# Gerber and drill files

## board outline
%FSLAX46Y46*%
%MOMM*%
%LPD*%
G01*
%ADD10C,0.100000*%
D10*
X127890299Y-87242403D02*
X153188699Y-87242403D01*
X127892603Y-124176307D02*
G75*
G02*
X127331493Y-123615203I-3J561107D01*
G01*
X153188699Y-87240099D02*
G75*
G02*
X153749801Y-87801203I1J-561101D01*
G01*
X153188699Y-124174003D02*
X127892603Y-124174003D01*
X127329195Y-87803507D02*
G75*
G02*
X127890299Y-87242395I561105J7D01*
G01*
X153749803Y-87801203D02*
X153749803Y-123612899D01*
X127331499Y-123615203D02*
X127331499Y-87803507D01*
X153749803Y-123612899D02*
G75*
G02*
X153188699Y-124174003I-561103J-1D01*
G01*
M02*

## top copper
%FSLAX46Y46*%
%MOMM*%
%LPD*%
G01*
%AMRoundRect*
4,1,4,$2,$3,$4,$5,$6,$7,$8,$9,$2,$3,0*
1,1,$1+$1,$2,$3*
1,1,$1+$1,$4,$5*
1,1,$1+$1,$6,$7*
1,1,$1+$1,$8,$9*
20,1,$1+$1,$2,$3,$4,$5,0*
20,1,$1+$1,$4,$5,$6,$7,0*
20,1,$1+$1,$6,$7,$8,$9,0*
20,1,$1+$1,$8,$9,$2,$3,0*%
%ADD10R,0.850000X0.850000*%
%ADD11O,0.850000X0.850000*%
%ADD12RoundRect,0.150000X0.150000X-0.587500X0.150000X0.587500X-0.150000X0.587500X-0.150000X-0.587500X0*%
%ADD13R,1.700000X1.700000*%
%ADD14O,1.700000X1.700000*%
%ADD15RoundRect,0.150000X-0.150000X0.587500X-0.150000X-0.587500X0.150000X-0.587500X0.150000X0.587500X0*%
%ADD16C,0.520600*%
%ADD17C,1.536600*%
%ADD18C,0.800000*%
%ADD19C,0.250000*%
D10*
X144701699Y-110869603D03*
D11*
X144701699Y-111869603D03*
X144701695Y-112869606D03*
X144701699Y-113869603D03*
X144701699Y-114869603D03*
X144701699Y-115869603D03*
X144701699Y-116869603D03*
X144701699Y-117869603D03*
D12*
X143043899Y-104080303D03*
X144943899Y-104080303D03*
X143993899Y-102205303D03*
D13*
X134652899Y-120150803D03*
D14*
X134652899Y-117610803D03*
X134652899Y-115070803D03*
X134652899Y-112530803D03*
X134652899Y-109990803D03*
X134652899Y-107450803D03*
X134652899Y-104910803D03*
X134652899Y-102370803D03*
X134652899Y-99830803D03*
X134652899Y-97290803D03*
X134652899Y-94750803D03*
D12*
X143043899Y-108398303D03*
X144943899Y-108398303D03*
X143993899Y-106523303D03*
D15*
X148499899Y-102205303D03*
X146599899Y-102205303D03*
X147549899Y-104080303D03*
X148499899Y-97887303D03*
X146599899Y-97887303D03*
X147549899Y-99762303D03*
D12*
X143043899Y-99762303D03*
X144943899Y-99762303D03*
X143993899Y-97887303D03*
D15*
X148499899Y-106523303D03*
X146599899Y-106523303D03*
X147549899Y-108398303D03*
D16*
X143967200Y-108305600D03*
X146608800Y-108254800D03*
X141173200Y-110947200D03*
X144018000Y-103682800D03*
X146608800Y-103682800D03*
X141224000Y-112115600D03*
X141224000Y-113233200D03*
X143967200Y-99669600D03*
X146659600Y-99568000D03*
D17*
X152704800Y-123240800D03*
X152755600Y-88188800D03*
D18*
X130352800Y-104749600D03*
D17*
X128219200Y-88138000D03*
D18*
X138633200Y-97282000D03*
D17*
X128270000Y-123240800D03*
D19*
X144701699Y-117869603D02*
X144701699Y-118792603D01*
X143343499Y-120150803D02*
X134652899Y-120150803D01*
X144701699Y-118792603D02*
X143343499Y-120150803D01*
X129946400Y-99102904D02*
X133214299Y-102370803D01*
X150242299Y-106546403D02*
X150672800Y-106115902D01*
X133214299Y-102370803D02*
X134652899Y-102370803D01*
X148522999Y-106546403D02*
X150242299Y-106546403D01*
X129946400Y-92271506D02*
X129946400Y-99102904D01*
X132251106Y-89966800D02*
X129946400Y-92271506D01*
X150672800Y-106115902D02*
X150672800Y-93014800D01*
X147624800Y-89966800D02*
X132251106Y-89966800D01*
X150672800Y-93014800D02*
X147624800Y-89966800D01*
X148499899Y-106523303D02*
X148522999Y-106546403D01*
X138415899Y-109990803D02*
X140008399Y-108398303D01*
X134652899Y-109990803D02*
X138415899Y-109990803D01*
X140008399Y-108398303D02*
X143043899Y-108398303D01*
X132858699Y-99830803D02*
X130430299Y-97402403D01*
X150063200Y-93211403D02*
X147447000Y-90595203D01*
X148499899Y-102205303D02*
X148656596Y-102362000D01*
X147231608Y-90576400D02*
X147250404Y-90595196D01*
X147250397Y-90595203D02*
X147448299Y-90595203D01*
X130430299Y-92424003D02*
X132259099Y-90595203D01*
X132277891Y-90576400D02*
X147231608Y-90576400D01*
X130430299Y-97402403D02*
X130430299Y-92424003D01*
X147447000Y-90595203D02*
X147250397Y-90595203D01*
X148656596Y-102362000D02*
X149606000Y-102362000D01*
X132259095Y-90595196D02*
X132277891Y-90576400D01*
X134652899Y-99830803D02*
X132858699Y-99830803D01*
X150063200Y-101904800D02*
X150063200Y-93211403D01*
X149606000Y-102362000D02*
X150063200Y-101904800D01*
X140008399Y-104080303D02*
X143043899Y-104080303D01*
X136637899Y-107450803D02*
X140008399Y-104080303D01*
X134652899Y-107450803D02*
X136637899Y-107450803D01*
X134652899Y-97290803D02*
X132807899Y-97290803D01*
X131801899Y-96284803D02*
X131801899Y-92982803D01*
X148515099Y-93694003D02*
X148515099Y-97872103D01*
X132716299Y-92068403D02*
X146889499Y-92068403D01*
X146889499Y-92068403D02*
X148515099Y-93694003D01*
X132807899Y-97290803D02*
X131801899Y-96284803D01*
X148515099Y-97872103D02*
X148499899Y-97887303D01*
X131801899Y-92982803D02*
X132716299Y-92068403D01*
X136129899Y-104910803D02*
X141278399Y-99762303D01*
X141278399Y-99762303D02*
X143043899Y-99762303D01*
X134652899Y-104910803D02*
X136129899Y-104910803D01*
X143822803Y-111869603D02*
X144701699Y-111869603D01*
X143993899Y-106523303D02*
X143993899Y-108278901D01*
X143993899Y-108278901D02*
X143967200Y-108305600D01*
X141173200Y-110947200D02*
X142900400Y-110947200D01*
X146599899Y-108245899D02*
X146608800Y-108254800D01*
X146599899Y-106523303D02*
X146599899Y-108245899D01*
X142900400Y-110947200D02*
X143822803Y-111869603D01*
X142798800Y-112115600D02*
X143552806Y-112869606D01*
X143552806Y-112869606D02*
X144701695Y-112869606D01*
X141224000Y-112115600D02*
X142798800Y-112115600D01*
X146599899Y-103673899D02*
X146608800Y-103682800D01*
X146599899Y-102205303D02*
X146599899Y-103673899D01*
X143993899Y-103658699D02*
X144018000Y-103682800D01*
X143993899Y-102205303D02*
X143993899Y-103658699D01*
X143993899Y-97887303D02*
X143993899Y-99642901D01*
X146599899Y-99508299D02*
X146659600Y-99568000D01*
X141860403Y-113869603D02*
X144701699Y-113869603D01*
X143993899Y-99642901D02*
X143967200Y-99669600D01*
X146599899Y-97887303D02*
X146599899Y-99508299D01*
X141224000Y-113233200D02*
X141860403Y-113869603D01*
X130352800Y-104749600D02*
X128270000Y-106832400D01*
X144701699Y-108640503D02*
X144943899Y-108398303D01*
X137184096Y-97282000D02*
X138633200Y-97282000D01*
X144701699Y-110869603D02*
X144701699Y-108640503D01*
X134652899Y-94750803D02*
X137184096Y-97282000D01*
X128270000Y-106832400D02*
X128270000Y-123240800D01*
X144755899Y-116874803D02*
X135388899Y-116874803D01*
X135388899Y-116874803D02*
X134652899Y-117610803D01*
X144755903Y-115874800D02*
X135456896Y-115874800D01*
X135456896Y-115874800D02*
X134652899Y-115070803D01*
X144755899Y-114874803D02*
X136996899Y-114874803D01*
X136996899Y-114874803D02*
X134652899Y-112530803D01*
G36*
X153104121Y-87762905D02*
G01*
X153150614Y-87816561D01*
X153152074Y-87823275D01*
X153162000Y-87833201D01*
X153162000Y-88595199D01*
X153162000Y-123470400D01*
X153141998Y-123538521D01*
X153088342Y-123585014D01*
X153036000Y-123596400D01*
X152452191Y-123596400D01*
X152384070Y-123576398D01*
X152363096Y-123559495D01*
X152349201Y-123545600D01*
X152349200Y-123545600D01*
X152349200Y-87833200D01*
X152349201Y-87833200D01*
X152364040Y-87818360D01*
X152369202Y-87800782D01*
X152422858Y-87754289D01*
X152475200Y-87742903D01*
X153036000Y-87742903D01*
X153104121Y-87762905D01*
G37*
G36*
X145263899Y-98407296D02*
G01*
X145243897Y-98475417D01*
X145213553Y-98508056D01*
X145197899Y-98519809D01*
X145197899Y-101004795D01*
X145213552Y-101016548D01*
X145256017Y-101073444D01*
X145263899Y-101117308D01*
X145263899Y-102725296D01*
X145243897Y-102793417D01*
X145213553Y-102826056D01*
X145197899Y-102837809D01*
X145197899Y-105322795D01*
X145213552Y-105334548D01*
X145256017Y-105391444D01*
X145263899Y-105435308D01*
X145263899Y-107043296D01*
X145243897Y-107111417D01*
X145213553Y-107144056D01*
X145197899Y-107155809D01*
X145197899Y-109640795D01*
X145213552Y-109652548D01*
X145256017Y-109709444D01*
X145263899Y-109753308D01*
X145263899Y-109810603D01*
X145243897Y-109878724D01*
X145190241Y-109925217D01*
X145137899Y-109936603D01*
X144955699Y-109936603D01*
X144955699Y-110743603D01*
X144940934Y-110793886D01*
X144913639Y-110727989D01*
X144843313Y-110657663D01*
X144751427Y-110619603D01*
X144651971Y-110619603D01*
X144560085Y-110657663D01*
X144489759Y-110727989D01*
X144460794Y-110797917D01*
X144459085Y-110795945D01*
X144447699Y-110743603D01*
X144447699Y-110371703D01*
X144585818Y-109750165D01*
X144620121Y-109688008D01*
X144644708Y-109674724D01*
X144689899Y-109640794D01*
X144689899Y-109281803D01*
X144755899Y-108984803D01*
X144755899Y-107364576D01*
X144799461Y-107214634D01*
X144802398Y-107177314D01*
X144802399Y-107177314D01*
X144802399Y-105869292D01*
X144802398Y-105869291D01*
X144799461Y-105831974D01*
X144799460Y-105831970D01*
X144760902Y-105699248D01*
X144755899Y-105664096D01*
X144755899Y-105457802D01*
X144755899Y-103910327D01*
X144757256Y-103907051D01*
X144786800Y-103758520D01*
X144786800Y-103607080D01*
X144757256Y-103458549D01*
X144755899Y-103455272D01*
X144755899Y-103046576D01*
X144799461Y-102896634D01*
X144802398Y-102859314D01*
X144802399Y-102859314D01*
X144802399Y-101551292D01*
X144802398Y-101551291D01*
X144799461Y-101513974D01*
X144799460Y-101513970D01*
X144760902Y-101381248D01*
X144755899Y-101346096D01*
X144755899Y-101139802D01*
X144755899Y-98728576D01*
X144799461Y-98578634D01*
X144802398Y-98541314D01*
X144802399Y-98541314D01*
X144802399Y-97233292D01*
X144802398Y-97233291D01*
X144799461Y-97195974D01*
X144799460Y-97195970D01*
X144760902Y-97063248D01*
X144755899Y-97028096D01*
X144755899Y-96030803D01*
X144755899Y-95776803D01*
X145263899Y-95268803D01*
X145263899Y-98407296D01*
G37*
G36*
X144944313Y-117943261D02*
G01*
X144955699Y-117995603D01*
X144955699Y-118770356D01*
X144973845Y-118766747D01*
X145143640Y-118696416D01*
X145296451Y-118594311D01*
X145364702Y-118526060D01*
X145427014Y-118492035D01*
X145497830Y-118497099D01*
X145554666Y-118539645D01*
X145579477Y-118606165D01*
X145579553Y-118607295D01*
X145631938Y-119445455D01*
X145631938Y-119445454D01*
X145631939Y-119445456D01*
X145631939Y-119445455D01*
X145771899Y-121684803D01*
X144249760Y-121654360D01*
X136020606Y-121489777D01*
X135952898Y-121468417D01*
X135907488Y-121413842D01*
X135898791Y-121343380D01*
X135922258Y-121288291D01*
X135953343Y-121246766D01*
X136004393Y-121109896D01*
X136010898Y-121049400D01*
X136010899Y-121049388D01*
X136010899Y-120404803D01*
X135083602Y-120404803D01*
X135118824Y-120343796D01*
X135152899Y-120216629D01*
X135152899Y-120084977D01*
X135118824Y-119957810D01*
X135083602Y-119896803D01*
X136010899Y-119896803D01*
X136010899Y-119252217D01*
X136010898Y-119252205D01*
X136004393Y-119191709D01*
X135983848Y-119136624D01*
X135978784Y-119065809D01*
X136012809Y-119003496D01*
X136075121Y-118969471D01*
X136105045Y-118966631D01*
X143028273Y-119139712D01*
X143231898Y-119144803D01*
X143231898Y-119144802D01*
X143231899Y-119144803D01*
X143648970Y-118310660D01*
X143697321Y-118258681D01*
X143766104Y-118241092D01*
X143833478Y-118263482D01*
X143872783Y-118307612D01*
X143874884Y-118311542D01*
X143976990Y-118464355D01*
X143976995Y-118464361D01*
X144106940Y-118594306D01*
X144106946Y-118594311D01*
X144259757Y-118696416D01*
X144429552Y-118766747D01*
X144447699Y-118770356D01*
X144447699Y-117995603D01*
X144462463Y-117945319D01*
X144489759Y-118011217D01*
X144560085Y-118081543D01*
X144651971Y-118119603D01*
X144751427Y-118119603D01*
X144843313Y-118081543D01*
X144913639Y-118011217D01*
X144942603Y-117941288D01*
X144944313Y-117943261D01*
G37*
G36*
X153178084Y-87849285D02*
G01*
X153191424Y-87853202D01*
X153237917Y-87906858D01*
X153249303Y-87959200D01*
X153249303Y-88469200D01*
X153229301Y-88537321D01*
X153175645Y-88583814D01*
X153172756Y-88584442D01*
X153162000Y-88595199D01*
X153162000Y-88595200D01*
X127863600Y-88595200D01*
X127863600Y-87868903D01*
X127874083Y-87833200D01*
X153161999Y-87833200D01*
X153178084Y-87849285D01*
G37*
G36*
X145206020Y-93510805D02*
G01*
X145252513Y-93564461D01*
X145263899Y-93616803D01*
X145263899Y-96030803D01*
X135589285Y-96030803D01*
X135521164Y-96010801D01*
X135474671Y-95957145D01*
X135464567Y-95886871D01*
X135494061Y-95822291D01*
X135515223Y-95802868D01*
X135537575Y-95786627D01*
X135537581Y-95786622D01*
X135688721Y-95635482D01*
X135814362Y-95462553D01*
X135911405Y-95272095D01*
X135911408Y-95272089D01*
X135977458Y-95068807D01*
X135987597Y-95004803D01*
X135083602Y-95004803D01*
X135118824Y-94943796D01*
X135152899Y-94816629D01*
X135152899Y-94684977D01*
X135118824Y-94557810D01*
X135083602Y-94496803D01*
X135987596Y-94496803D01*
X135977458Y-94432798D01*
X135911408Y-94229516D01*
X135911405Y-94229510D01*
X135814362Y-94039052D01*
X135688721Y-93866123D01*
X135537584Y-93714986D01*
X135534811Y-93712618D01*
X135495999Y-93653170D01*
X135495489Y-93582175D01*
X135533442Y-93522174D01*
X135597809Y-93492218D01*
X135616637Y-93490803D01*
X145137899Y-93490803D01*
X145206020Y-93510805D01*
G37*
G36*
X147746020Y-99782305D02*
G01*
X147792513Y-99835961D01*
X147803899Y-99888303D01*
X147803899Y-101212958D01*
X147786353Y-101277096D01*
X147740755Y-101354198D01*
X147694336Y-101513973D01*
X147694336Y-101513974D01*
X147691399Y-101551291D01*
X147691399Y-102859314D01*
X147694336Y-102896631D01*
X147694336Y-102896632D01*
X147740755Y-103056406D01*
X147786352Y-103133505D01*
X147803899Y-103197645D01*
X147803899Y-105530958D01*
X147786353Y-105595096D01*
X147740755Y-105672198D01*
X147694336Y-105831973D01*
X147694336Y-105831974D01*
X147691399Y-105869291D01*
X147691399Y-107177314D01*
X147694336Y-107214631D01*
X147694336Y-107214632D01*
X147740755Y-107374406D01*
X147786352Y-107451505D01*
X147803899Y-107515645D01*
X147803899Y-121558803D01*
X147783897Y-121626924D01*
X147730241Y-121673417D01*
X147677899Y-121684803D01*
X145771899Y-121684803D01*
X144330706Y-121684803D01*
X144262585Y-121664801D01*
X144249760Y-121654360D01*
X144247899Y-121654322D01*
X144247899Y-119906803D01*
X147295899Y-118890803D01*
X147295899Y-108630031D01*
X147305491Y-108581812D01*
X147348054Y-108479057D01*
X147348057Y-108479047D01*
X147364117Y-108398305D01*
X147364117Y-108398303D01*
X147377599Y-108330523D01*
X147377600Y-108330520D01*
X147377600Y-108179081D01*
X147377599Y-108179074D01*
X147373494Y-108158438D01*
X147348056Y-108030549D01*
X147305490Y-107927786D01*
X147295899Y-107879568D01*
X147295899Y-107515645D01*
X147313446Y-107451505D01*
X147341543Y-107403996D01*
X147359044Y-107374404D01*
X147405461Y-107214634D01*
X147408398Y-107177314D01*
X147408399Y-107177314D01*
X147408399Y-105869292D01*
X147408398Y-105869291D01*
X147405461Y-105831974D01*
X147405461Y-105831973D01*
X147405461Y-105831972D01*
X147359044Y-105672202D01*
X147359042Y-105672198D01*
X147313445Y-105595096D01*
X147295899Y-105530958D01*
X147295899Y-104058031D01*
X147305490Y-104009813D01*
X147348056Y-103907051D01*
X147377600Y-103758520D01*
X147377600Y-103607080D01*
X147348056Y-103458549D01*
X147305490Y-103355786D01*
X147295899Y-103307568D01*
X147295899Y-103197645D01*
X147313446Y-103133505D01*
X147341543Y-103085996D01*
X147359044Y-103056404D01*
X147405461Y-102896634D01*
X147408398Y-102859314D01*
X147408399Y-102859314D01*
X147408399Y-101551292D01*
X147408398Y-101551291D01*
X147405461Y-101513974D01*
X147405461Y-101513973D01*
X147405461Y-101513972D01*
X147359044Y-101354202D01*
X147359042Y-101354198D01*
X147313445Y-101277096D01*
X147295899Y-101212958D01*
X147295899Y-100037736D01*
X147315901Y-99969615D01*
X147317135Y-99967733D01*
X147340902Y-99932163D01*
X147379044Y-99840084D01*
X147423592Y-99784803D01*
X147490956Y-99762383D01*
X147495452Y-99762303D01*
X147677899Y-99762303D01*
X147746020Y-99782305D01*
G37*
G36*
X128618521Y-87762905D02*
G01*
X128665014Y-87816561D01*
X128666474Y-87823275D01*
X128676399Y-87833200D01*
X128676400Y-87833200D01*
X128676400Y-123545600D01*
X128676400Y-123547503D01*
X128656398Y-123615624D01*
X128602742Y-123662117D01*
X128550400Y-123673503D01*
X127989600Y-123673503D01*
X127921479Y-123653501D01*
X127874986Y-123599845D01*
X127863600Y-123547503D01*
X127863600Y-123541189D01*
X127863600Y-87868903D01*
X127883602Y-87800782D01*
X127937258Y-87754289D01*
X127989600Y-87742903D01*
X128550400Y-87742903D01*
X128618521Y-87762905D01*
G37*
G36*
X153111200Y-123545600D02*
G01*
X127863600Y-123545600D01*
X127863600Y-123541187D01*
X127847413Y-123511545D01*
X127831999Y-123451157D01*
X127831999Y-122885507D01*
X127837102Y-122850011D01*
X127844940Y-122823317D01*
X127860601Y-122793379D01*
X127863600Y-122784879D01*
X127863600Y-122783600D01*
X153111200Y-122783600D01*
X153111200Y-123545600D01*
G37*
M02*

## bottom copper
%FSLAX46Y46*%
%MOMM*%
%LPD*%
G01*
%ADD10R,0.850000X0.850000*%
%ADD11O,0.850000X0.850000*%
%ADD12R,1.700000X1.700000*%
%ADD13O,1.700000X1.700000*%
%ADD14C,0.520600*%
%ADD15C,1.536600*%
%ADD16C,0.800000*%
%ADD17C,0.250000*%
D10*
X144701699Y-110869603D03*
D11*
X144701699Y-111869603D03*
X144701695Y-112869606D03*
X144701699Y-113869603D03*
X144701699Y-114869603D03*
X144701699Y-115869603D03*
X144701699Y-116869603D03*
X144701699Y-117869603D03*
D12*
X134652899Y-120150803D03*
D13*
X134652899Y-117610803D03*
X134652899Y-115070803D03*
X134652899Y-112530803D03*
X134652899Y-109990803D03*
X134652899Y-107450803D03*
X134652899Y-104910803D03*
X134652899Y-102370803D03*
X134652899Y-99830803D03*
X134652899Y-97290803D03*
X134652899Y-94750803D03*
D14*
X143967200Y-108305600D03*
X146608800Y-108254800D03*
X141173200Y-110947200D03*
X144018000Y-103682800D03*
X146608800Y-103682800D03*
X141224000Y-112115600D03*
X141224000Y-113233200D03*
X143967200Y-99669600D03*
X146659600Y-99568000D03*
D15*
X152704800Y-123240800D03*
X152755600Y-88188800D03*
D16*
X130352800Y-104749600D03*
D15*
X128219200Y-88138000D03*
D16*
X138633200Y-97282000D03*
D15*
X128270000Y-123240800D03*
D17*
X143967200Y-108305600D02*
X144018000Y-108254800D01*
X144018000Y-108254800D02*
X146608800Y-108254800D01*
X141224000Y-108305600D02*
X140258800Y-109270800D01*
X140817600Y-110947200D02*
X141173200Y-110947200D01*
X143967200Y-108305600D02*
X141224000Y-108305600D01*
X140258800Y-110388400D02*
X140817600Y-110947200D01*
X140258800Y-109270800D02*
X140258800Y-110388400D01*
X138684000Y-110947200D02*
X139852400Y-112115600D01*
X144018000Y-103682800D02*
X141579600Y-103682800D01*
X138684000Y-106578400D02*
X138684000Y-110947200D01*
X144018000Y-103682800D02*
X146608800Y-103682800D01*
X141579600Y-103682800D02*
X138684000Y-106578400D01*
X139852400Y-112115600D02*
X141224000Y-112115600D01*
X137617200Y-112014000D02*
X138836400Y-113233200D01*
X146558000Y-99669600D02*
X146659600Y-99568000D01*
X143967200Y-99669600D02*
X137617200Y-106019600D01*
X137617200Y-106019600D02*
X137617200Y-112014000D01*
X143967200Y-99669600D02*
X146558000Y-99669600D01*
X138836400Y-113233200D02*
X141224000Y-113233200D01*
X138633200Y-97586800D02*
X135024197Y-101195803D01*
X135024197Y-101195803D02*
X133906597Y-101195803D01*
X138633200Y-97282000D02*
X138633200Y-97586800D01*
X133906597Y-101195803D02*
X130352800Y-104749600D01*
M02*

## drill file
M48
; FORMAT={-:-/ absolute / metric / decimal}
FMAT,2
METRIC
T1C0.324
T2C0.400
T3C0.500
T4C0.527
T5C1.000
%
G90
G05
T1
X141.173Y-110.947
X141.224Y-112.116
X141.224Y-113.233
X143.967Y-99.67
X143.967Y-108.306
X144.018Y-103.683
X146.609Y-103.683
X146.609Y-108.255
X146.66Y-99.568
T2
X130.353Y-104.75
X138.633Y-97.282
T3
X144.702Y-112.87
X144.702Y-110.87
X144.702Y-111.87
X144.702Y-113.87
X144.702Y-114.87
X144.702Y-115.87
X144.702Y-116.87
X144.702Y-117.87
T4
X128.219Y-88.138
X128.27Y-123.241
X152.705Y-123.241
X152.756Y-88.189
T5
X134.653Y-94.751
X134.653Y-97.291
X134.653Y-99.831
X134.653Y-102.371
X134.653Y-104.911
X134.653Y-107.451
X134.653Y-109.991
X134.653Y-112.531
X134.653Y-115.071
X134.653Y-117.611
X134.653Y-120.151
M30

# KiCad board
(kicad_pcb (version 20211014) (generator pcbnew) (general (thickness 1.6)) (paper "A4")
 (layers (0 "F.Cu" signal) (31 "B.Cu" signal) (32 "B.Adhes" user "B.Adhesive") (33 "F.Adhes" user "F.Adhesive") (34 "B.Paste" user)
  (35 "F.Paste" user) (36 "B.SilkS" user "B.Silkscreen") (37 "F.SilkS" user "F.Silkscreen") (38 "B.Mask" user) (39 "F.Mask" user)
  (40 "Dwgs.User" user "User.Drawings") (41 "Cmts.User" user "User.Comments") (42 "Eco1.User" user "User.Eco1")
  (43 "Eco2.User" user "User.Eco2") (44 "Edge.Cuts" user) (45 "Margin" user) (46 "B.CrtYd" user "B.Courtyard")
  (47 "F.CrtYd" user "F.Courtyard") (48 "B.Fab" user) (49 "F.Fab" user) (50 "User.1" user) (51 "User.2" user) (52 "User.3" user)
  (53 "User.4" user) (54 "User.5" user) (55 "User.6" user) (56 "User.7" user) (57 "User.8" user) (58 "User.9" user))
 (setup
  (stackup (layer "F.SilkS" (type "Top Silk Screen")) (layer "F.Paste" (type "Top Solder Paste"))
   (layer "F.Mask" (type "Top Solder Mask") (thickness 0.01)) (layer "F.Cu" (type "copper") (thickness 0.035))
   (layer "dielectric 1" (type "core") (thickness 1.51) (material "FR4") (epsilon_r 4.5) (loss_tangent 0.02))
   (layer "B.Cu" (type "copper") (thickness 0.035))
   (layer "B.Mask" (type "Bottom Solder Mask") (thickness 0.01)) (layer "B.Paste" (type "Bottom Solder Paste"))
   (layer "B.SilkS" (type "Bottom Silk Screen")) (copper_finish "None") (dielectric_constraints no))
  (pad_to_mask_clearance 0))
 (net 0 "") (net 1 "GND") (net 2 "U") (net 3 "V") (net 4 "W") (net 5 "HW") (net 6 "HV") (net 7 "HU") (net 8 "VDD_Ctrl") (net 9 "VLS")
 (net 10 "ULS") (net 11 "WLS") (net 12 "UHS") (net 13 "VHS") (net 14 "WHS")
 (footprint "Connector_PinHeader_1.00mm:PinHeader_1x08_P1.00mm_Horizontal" (layer "F.Cu") (at 144.701699 110.869603)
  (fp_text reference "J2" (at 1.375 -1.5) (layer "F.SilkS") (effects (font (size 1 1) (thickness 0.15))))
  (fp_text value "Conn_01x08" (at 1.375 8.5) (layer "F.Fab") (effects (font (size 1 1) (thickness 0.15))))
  (pad "1" thru_hole rect (at 0 0) (size 0.85 0.85) (drill 0.5) (layers *.Cu *.Mask) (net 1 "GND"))
  (pad "2" thru_hole oval (at 0 1) (size 0.85 0.85) (drill 0.5) (layers *.Cu *.Mask) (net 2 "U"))
  (pad "3" thru_hole oval (at -0.000004 2.000003) (size 0.85 0.85) (drill 0.5) (layers *.Cu *.Mask) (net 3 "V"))
  (pad "4" thru_hole oval (at 0 3) (size 0.85 0.85) (drill 0.5) (layers *.Cu *.Mask) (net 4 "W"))
  (pad "5" thru_hole oval (at 0 4) (size 0.85 0.85) (drill 0.5) (layers *.Cu *.Mask) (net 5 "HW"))
  (pad "6" thru_hole oval (at 0 5) (size 0.85 0.85) (drill 0.5) (layers *.Cu *.Mask) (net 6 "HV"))
  (pad "7" thru_hole oval (at 0 6) (size 0.85 0.85) (drill 0.5) (layers *.Cu *.Mask) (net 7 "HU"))
  (pad "8" thru_hole oval (at 0 7) (size 0.85 0.85) (drill 0.5) (layers *.Cu *.Mask) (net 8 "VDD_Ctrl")))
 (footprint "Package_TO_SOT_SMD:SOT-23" (layer "F.Cu") (at 143.993899 103.142803 90)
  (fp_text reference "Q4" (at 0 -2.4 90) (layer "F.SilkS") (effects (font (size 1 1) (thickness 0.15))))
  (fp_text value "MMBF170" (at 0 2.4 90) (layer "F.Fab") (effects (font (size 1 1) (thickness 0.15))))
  (pad "1" smd roundrect (at -0.9375 -0.95 90) (size 1.475 0.6) (layers "F.Cu" "F.Paste" "F.Mask") (roundrect_rratio 0.25) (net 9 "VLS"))
  (pad "2" smd roundrect (at -0.9375 0.95 90) (size 1.475 0.6) (layers "F.Cu" "F.Paste" "F.Mask") (roundrect_rratio 0.25) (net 1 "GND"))
  (pad "3" smd roundrect (at 0.9375 0 90) (size 1.475 0.6) (layers "F.Cu" "F.Paste" "F.Mask") (roundrect_rratio 0.25) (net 3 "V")))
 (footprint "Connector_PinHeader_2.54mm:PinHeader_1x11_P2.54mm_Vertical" (layer "F.Cu") (at 134.652899 120.150803 180)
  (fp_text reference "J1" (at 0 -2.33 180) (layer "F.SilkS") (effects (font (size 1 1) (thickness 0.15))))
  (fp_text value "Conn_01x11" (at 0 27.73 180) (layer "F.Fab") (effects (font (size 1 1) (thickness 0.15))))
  (pad "1" thru_hole rect (at 0 0 180) (size 1.7 1.7) (drill 1) (layers *.Cu *.Mask) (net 8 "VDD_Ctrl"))
  (pad "2" thru_hole oval (at 0 2.54 180) (size 1.7 1.7) (drill 1) (layers *.Cu *.Mask) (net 7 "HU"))
  (pad "3" thru_hole oval (at 0 5.08 180) (size 1.7 1.7) (drill 1) (layers *.Cu *.Mask) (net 6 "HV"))
  (pad "4" thru_hole oval (at 0 7.62 180) (size 1.7 1.7) (drill 1) (layers *.Cu *.Mask) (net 5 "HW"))
  (pad "5" thru_hole oval (at 0 10.16 180) (size 1.7 1.7) (drill 1) (layers *.Cu *.Mask) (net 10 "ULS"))
  (pad "6" thru_hole oval (at 0 12.7 180) (size 1.7 1.7) (drill 1) (layers *.Cu *.Mask) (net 9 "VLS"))
  (pad "7" thru_hole oval (at 0 15.24 180) (size 1.7 1.7) (drill 1) (layers *.Cu *.Mask) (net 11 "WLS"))
  (pad "8" thru_hole oval (at 0 17.78 180) (size 1.7 1.7) (drill 1) (layers *.Cu *.Mask) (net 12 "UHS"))
  (pad "9" thru_hole oval (at 0 20.32 180) (size 1.7 1.7) (drill 1) (layers *.Cu *.Mask) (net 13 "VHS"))
  (pad "10" thru_hole oval (at 0 22.86 180) (size 1.7 1.7) (drill 1) (layers *.Cu *.Mask) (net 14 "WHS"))
  (pad "11" thru_hole oval (at 0 25.4 180) (size 1.7 1.7) (drill 1) (layers *.Cu *.Mask) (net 1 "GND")))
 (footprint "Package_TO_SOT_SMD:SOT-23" (layer "F.Cu") (at 143.993899 107.460803 90)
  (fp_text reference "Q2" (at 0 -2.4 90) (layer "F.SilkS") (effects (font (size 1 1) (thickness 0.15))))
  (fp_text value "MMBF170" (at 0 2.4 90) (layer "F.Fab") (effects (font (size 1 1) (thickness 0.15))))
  (pad "1" smd roundrect (at -0.9375 -0.95 90) (size 1.475 0.6) (layers "F.Cu" "F.Paste" "F.Mask") (roundrect_rratio 0.25) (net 10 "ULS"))
  (pad "2" smd roundrect (at -0.9375 0.95 90) (size 1.475 0.6) (layers "F.Cu" "F.Paste" "F.Mask") (roundrect_rratio 0.25) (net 1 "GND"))
  (pad "3" smd roundrect (at 0.9375 0 90) (size 1.475 0.6) (layers "F.Cu" "F.Paste" "F.Mask") (roundrect_rratio 0.25) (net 2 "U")))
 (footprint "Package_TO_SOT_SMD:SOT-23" (layer "F.Cu") (at 147.549899 103.142803 -90)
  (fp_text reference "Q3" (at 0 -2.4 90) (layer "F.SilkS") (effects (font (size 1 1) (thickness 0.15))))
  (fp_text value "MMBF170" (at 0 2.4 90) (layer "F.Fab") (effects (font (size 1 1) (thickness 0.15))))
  (pad "1" smd roundrect (at -0.9375 -0.95 270) (size 1.475 0.6) (layers "F.Cu" "F.Paste" "F.Mask") (roundrect_rratio 0.25) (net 13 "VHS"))
  (pad "2" smd roundrect (at -0.9375 0.95 270) (size 1.475 0.6) (layers "F.Cu" "F.Paste" "F.Mask") (roundrect_rratio 0.25) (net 3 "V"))
  (pad "3" smd roundrect (at 0.9375 0 270) (size 1.475 0.6) (layers "F.Cu" "F.Paste" "F.Mask") (roundrect_rratio 0.25) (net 8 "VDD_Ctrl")))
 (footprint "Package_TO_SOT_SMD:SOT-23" (layer "F.Cu") (at 147.549899 98.824803 -90)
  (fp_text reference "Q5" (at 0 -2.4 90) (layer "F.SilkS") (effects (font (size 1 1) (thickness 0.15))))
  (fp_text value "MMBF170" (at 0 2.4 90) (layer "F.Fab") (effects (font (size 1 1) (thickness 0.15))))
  (pad "1" smd roundrect (at -0.9375 -0.95 270) (size 1.475 0.6) (layers "F.Cu" "F.Paste" "F.Mask") (roundrect_rratio 0.25) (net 14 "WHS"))
  (pad "2" smd roundrect (at -0.9375 0.95 270) (size 1.475 0.6) (layers "F.Cu" "F.Paste" "F.Mask") (roundrect_rratio 0.25) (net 4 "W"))
  (pad "3" smd roundrect (at 0.9375 0 270) (size 1.475 0.6) (layers "F.Cu" "F.Paste" "F.Mask") (roundrect_rratio 0.25) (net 8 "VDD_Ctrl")))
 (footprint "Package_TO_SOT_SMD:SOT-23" (layer "F.Cu") (at 143.993899 98.824803 90)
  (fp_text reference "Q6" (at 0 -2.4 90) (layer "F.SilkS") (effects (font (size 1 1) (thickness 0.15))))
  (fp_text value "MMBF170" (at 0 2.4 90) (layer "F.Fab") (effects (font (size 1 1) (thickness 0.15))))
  (pad "1" smd roundrect (at -0.9375 -0.95 90) (size 1.475 0.6) (layers "F.Cu" "F.Paste" "F.Mask") (roundrect_rratio 0.25) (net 11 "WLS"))
  (pad "2" smd roundrect (at -0.9375 0.95 90) (size 1.475 0.6) (layers "F.Cu" "F.Paste" "F.Mask") (roundrect_rratio 0.25) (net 1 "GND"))
  (pad "3" smd roundrect (at 0.9375 0 90) (size 1.475 0.6) (layers "F.Cu" "F.Paste" "F.Mask") (roundrect_rratio 0.25) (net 4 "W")))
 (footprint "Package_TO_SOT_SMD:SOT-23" (layer "F.Cu") (at 147.549899 107.460803 -90)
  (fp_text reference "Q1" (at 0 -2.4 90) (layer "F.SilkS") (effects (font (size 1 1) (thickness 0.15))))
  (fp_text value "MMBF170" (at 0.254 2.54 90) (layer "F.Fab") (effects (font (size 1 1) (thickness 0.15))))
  (pad "1" smd roundrect (at -0.9375 -0.95 270) (size 1.475 0.6) (layers "F.Cu" "F.Paste" "F.Mask") (roundrect_rratio 0.25) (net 12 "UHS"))
  (pad "2" smd roundrect (at -0.9375 0.95 270) (size 1.475 0.6) (layers "F.Cu" "F.Paste" "F.Mask") (roundrect_rratio 0.25) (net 2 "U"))
  (pad "3" smd roundrect (at 0.9375 0 270) (size 1.475 0.6) (layers "F.Cu" "F.Paste" "F.Mask") (roundrect_rratio 0.25) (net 8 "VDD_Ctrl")))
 (gr_line (start 127.890299 87.242403) (end 153.188699 87.242403) (layer "Edge.Cuts") (width 0.1))
 (gr_arc (start 127.892603 124.176307) (mid 127.495843 124.011963) (end 127.331499 123.615203) (layer "Edge.Cuts") (width 0.1))
 (gr_arc (start 153.188699 87.240099) (mid 153.585459 87.404443) (end 153.749803 87.801203) (layer "Edge.Cuts") (width 0.1))
 (gr_line (start 153.188699 124.174003) (end 127.892603 124.174003) (layer "Edge.Cuts") (width 0.1))
 (gr_arc (start 127.329195 87.803507) (mid 127.493539 87.406747) (end 127.890299 87.242403) (layer "Edge.Cuts") (width 0.1))
 (gr_line (start 153.749803 87.801203) (end 153.749803 123.612899) (layer "Edge.Cuts") (width 0.1))
 (gr_line (start 127.331499 123.615203) (end 127.331499 87.803507) (layer "Edge.Cuts") (width 0.1))
 (gr_arc (start 153.749803 123.612899) (mid 153.585459 124.009659) (end 153.188699 124.174003) (layer "Edge.Cuts") (width 0.1))
 (segment (start 144.701699 117.869603) (end 144.701699 118.792603) (width 0.25) (layer "F.Cu") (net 8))
 (segment (start 143.343499 120.150803) (end 134.652899 120.150803) (width 0.25) (layer "F.Cu") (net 8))
 (segment (start 144.701699 118.792603) (end 143.343499 120.150803) (width 0.25) (layer "F.Cu") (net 8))
 (segment (start 129.9464 99.102904) (end 133.214299 102.370803) (width 0.25) (layer "F.Cu") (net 12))
 (segment (start 150.242299 106.546403) (end 150.6728 106.115902) (width 0.25) (layer "F.Cu") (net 12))
 (segment (start 133.214299 102.370803) (end 134.652899 102.370803) (width 0.25) (layer "F.Cu") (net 12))
 (segment (start 148.522999 106.546403) (end 150.242299 106.546403) (width 0.25) (layer "F.Cu") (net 12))
 (segment (start 129.9464 92.271506) (end 129.9464 99.102904) (width 0.25) (layer "F.Cu") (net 12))
 (segment (start 132.251106 89.9668) (end 129.9464 92.271506) (width 0.25) (layer "F.Cu") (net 12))
 (segment (start 150.6728 106.115902) (end 150.6728 93.0148) (width 0.25) (layer "F.Cu") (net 12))
 (segment (start 147.6248 89.9668) (end 132.251106 89.9668) (width 0.25) (layer "F.Cu") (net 12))
 (segment (start 150.6728 93.0148) (end 147.6248 89.9668) (width 0.25) (layer "F.Cu") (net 12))
 (segment (start 148.499899 106.523303) (end 148.522999 106.546403) (width 0.25) (layer "F.Cu") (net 12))
 (segment (start 138.415899 109.990803) (end 140.008399 108.398303) (width 0.25) (layer "F.Cu") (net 10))
 (segment (start 134.652899 109.990803) (end 138.415899 109.990803) (width 0.25) (layer "F.Cu") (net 10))
 (segment (start 140.008399 108.398303) (end 143.043899 108.398303) (width 0.25) (layer "F.Cu") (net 10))
 (segment (start 132.858699 99.830803) (end 130.430299 97.402403) (width 0.25) (layer "F.Cu") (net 13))
 (segment (start 150.0632 93.211403) (end 147.447 90.595203) (width 0.25) (layer "F.Cu") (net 13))
 (segment (start 148.499899 102.205303) (end 148.656596 102.362) (width 0.25) (layer "F.Cu") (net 13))
 (segment (start 147.231608 90.5764) (end 147.250404 90.595196) (width 0.25) (layer "F.Cu") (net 13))
 (segment (start 147.250397 90.595203) (end 147.448299 90.595203) (width 0.25) (layer "F.Cu") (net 13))
 (segment (start 130.430299 92.424003) (end 132.259099 90.595203) (width 0.25) (layer "F.Cu") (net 13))
 (segment (start 132.277891 90.5764) (end 147.231608 90.5764) (width 0.25) (layer "F.Cu") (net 13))
 (segment (start 130.430299 97.402403) (end 130.430299 92.424003) (width 0.25) (layer "F.Cu") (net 13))
 (segment (start 147.447 90.595203) (end 147.250397 90.595203) (width 0.25) (layer "F.Cu") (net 13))
 (segment (start 148.656596 102.362) (end 149.606 102.362) (width 0.25) (layer "F.Cu") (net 13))
 (segment (start 132.259095 90.595196) (end 132.277891 90.5764) (width 0.25) (layer "F.Cu") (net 13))
 (segment (start 134.652899 99.830803) (end 132.858699 99.830803) (width 0.25) (layer "F.Cu") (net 13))
 (segment (start 150.0632 101.9048) (end 150.0632 93.211403) (width 0.25) (layer "F.Cu") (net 13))
 (segment (start 149.606 102.362) (end 150.0632 101.9048) (width 0.25) (layer "F.Cu") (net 13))
 (segment (start 140.008399 104.080303) (end 143.043899 104.080303) (width 0.25) (layer "F.Cu") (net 9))
 (segment (start 136.637899 107.450803) (end 140.008399 104.080303) (width 0.25) (layer "F.Cu") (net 9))
 (segment (start 134.652899 107.450803) (end 136.637899 107.450803) (width 0.25) (layer "F.Cu") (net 9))
 (segment (start 134.652899 97.290803) (end 132.807899 97.290803) (width 0.25) (layer "F.Cu") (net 14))
 (segment (start 131.801899 96.284803) (end 131.801899 92.982803) (width 0.25) (layer "F.Cu") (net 14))
 (segment (start 148.515099 93.694003) (end 148.515099 97.872103) (width 0.25) (layer "F.Cu") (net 14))
 (segment (start 132.716299 92.068403) (end 146.889499 92.068403) (width 0.25) (layer "F.Cu") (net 14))
 (segment (start 146.889499 92.068403) (end 148.515099 93.694003) (width 0.25) (layer "F.Cu") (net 14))
 (segment (start 132.807899 97.290803) (end 131.801899 96.284803) (width 0.25) (layer "F.Cu") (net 14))
 (segment (start 148.515099 97.872103) (end 148.499899 97.887303) (width 0.25) (layer "F.Cu") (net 14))
 (segment (start 131.801899 92.982803) (end 132.716299 92.068403) (width 0.25) (layer "F.Cu") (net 14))
 (segment (start 136.129899 104.910803) (end 141.278399 99.762303) (width 0.25) (layer "F.Cu") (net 11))
 (segment (start 141.278399 99.762303) (end 143.043899 99.762303) (width 0.25) (layer "F.Cu") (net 11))
 (segment (start 134.652899 104.910803) (end 136.129899 104.910803) (width 0.25) (layer "F.Cu") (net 11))
 (segment (start 143.822803 111.869603) (end 144.701699 111.869603) (width 0.25) (layer "F.Cu") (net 2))
 (segment (start 143.993899 106.523303) (end 143.993899 108.278901) (width 0.25) (layer "F.Cu") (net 2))
 (segment (start 143.993899 108.278901) (end 143.9672 108.3056) (width 0.25) (layer "F.Cu") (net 2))
 (segment (start 141.1732 110.9472) (end 142.9004 110.9472) (width 0.25) (layer "F.Cu") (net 2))
 (segment (start 146.599899 108.245899) (end 146.6088 108.2548) (width 0.25) (layer "F.Cu") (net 2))
 (segment (start 146.599899 106.523303) (end 146.599899 108.245899) (width 0.25) (layer "F.Cu") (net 2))
 (segment (start 142.9004 110.9472) (end 143.822803 111.869603) (width 0.25) (layer "F.Cu") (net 2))
 (via (at 143.9672 108.3056) (size 0.5206) (drill 0.3238) (layers "F.Cu" "B.Cu") (free) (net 2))
 (via (at 146.6088 108.2548) (size 0.5206) (drill 0.3238) (layers "F.Cu" "B.Cu") (free) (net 2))
 (via (at 141.1732 110.9472) (size 0.5206) (drill 0.3238) (layers "F.Cu" "B.Cu") (free) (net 2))
 (segment (start 143.9672 108.3056) (end 144.018 108.2548) (width 0.25) (layer "B.Cu") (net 2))
 (segment (start 144.018 108.2548) (end 146.6088 108.2548) (width 0.25) (layer "B.Cu") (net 2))
 (segment (start 141.224 108.3056) (end 140.2588 109.2708) (width 0.25) (layer "B.Cu") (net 2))
 (segment (start 140.8176 110.9472) (end 141.1732 110.9472) (width 0.25) (layer "B.Cu") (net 2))
 (segment (start 143.9672 108.3056) (end 141.224 108.3056) (width 0.25) (layer "B.Cu") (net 2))
 (segment (start 140.2588 110.3884) (end 140.8176 110.9472) (width 0.25) (layer "B.Cu") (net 2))
 (segment (start 140.2588 109.2708) (end 140.2588 110.3884) (width 0.25) (layer "B.Cu") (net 2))
 (segment (start 142.7988 112.1156) (end 143.552806 112.869606) (width 0.25) (layer "F.Cu") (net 3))
 (segment (start 143.552806 112.869606) (end 144.701695 112.869606) (width 0.25) (layer "F.Cu") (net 3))
 (segment (start 141.224 112.1156) (end 142.7988 112.1156) (width 0.25) (layer "F.Cu") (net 3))
 (segment (start 146.599899 103.673899) (end 146.6088 103.6828) (width 0.25) (layer "F.Cu") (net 3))
 (segment (start 146.599899 102.205303) (end 146.599899 103.673899) (width 0.25) (layer "F.Cu") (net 3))
 (segment (start 143.993899 103.658699) (end 144.018 103.6828) (width 0.25) (layer "F.Cu") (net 3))
 (segment (start 143.993899 102.205303) (end 143.993899 103.658699) (width 0.25) (layer "F.Cu") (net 3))
 (via (at 144.018 103.6828) (size 0.5206) (drill 0.3238) (layers "F.Cu" "B.Cu") (free) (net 3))
 (via (at 146.6088 103.6828) (size 0.5206) (drill 0.3238) (layers "F.Cu" "B.Cu") (free) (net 3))
 (via (at 141.224 112.1156) (size 0.5206) (drill 0.3238) (layers "F.Cu" "B.Cu") (free) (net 3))
 (segment (start 138.684 110.9472) (end 139.8524 112.1156) (width 0.25) (layer "B.Cu") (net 3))
 (segment (start 144.018 103.6828) (end 141.5796 103.6828) (width 0.25) (layer "B.Cu") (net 3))
 (segment (start 138.684 106.5784) (end 138.684 110.9472) (width 0.25) (layer "B.Cu") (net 3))
 (segment (start 144.018 103.6828) (end 146.6088 103.6828) (width 0.25) (layer "B.Cu") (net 3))
 (segment (start 141.5796 103.6828) (end 138.684 106.5784) (width 0.25) (layer "B.Cu") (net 3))
 (segment (start 139.8524 112.1156) (end 141.224 112.1156) (width 0.25) (layer "B.Cu") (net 3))
 (segment (start 143.993899 97.887303) (end 143.993899 99.642901) (width 0.25) (layer "F.Cu") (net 4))
 (segment (start 146.599899 99.508299) (end 146.6596 99.568) (width 0.25) (layer "F.Cu") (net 4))
 (segment (start 141.860403 113.869603) (end 144.701699 113.869603) (width 0.25) (layer "F.Cu") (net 4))
 (segment (start 143.993899 99.642901) (end 143.9672 99.6696) (width 0.25) (layer "F.Cu") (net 4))
 (segment (start 146.599899 97.887303) (end 146.599899 99.508299) (width 0.25) (layer "F.Cu") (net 4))
 (segment (start 141.224 113.2332) (end 141.860403 113.869603) (width 0.25) (layer "F.Cu") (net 4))
 (via (at 141.224 113.2332) (size 0.5206) (drill 0.3238) (layers "F.Cu" "B.Cu") (free) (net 4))
 (via (at 143.9672 99.6696) (size 0.5206) (drill 0.3238) (layers "F.Cu" "B.Cu") (free) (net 4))
 (via (at 146.6596 99.568) (size 0.5206) (drill 0.3238) (layers "F.Cu" "B.Cu") (free) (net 4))
 (segment (start 137.6172 112.014) (end 138.8364 113.2332) (width 0.25) (layer "B.Cu") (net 4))
 (segment (start 146.558 99.6696) (end 146.6596 99.568) (width 0.25) (layer "B.Cu") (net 4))
 (segment (start 143.9672 99.6696) (end 137.6172 106.0196) (width 0.25) (layer "B.Cu") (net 4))
 (segment (start 137.6172 106.0196) (end 137.6172 112.014) (width 0.25) (layer "B.Cu") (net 4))
 (segment (start 143.9672 99.6696) (end 146.558 99.6696) (width 0.25) (layer "B.Cu") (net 4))
 (segment (start 138.8364 113.2332) (end 141.224 113.2332) (width 0.25) (layer "B.Cu") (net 4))
 (segment (start 130.3528 104.7496) (end 128.27 106.8324) (width 0.25) (layer "F.Cu") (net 1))
 (segment (start 144.701699 108.640503) (end 144.943899 108.398303) (width 0.25) (layer "F.Cu") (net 1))
 (segment (start 137.184096 97.282) (end 138.6332 97.282) (width 0.25) (layer "F.Cu") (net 1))
 (segment (start 144.701699 110.869603) (end 144.701699 108.640503) (width 0.25) (layer "F.Cu") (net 1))
 (segment (start 134.652899 94.750803) (end 137.184096 97.282) (width 0.25) (layer "F.Cu") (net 1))
 (segment (start 128.27 106.8324) (end 128.27 123.2408) (width 0.25) (layer "F.Cu") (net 1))
 (via (at 152.7048 123.2408) (size 1.5366) (drill 0.527) (layers "F.Cu" "B.Cu") (free) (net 1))
 (via (at 152.7556 88.1888) (size 1.5366) (drill 0.527) (layers "F.Cu" "B.Cu") (free) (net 1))
 (via (at 130.3528 104.7496) (size 0.8) (drill 0.4) (layers "F.Cu" "B.Cu") (free) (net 1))
 (via (at 128.2192 88.138) (size 1.5366) (drill 0.527) (layers "F.Cu" "B.Cu") (free) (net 1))
 (via (at 138.6332 97.282) (size 0.8) (drill 0.4) (layers "F.Cu" "B.Cu") (free) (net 1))
 (via (at 128.27 123.2408) (size 1.5366) (drill 0.527) (layers "F.Cu" "B.Cu") (free) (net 1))
 (segment (start 138.6332 97.5868) (end 135.024197 101.195803) (width 0.25) (layer "B.Cu") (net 1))
 (segment (start 135.024197 101.195803) (end 133.906597 101.195803) (width 0.25) (layer "B.Cu") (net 1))
 (segment (start 138.6332 97.282) (end 138.6332 97.5868) (width 0.25) (layer "B.Cu") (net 1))
 (segment (start 133.906597 101.195803) (end 130.3528 104.7496) (width 0.25) (layer "B.Cu") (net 1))
 (segment (start 144.755899 116.874803) (end 135.388899 116.874803) (width 0.25) (layer "F.Cu") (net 7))
 (segment (start 135.388899 116.874803) (end 134.652899 117.610803) (width 0.25) (layer "F.Cu") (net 7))
 (segment (start 144.755903 115.8748) (end 135.456896 115.8748) (width 0.25) (layer "F.Cu") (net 6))
 (segment (start 135.456896 115.8748) (end 134.652899 115.070803) (width 0.25) (layer "F.Cu") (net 6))
 (segment (start 144.755899 114.874803) (end 136.996899 114.874803) (width 0.25) (layer "F.Cu") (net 5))
 (segment (start 136.996899 114.874803) (end 134.652899 112.530803) (width 0.25) (layer "F.Cu") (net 5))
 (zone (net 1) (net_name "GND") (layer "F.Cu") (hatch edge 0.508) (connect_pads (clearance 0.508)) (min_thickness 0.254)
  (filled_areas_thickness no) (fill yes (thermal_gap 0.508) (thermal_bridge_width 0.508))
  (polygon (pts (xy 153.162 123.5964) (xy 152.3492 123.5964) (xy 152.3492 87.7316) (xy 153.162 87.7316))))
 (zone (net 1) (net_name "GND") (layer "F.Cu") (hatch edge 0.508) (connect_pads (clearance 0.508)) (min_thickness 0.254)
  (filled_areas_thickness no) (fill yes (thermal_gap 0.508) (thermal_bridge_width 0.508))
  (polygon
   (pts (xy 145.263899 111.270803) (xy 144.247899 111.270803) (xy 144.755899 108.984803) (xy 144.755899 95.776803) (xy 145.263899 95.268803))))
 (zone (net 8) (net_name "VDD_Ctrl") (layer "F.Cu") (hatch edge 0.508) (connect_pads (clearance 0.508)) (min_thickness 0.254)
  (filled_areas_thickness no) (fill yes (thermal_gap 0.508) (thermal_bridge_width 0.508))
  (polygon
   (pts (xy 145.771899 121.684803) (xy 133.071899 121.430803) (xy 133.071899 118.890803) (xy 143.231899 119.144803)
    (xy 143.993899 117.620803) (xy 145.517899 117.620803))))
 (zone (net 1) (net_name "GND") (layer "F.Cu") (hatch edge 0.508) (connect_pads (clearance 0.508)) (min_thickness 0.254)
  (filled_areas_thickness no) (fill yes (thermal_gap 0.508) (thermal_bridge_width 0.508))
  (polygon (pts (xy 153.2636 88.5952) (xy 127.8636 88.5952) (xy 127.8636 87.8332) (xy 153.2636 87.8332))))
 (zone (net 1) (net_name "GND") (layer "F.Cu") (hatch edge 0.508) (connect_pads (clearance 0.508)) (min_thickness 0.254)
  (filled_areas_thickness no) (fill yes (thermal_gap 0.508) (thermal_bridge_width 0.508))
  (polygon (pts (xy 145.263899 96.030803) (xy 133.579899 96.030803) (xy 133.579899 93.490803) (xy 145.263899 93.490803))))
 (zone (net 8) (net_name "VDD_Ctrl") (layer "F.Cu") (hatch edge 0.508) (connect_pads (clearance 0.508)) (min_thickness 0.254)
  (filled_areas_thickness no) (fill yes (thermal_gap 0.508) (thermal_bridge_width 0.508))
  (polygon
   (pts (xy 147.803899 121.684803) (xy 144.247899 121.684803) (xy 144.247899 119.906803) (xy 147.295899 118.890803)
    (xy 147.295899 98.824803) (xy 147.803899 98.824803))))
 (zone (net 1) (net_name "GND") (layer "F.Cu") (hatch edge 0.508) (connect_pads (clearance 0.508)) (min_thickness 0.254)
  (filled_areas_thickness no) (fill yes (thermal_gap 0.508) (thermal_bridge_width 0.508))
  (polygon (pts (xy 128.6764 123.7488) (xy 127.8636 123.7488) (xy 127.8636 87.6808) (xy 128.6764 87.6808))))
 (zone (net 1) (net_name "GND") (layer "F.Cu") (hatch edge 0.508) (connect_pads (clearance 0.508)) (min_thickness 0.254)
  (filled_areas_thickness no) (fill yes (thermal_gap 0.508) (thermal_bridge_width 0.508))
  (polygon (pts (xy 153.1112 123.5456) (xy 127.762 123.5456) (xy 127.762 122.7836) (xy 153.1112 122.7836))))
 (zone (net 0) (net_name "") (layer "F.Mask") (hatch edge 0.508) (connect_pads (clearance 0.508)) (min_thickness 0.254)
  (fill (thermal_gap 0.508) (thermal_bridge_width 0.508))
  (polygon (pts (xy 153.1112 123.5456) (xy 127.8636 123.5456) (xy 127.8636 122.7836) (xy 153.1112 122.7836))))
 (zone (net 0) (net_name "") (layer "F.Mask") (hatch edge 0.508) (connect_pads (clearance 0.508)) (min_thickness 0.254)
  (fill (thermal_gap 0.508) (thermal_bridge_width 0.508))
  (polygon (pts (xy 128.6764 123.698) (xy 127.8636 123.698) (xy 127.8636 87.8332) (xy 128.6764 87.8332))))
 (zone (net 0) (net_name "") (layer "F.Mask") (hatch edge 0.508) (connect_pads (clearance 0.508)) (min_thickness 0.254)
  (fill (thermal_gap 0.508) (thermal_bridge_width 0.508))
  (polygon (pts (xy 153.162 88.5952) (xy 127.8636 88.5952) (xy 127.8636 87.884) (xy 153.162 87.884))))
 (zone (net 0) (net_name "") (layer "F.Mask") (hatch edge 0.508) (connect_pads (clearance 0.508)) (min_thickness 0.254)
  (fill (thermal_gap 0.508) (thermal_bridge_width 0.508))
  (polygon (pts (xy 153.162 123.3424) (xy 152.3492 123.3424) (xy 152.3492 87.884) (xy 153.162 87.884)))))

